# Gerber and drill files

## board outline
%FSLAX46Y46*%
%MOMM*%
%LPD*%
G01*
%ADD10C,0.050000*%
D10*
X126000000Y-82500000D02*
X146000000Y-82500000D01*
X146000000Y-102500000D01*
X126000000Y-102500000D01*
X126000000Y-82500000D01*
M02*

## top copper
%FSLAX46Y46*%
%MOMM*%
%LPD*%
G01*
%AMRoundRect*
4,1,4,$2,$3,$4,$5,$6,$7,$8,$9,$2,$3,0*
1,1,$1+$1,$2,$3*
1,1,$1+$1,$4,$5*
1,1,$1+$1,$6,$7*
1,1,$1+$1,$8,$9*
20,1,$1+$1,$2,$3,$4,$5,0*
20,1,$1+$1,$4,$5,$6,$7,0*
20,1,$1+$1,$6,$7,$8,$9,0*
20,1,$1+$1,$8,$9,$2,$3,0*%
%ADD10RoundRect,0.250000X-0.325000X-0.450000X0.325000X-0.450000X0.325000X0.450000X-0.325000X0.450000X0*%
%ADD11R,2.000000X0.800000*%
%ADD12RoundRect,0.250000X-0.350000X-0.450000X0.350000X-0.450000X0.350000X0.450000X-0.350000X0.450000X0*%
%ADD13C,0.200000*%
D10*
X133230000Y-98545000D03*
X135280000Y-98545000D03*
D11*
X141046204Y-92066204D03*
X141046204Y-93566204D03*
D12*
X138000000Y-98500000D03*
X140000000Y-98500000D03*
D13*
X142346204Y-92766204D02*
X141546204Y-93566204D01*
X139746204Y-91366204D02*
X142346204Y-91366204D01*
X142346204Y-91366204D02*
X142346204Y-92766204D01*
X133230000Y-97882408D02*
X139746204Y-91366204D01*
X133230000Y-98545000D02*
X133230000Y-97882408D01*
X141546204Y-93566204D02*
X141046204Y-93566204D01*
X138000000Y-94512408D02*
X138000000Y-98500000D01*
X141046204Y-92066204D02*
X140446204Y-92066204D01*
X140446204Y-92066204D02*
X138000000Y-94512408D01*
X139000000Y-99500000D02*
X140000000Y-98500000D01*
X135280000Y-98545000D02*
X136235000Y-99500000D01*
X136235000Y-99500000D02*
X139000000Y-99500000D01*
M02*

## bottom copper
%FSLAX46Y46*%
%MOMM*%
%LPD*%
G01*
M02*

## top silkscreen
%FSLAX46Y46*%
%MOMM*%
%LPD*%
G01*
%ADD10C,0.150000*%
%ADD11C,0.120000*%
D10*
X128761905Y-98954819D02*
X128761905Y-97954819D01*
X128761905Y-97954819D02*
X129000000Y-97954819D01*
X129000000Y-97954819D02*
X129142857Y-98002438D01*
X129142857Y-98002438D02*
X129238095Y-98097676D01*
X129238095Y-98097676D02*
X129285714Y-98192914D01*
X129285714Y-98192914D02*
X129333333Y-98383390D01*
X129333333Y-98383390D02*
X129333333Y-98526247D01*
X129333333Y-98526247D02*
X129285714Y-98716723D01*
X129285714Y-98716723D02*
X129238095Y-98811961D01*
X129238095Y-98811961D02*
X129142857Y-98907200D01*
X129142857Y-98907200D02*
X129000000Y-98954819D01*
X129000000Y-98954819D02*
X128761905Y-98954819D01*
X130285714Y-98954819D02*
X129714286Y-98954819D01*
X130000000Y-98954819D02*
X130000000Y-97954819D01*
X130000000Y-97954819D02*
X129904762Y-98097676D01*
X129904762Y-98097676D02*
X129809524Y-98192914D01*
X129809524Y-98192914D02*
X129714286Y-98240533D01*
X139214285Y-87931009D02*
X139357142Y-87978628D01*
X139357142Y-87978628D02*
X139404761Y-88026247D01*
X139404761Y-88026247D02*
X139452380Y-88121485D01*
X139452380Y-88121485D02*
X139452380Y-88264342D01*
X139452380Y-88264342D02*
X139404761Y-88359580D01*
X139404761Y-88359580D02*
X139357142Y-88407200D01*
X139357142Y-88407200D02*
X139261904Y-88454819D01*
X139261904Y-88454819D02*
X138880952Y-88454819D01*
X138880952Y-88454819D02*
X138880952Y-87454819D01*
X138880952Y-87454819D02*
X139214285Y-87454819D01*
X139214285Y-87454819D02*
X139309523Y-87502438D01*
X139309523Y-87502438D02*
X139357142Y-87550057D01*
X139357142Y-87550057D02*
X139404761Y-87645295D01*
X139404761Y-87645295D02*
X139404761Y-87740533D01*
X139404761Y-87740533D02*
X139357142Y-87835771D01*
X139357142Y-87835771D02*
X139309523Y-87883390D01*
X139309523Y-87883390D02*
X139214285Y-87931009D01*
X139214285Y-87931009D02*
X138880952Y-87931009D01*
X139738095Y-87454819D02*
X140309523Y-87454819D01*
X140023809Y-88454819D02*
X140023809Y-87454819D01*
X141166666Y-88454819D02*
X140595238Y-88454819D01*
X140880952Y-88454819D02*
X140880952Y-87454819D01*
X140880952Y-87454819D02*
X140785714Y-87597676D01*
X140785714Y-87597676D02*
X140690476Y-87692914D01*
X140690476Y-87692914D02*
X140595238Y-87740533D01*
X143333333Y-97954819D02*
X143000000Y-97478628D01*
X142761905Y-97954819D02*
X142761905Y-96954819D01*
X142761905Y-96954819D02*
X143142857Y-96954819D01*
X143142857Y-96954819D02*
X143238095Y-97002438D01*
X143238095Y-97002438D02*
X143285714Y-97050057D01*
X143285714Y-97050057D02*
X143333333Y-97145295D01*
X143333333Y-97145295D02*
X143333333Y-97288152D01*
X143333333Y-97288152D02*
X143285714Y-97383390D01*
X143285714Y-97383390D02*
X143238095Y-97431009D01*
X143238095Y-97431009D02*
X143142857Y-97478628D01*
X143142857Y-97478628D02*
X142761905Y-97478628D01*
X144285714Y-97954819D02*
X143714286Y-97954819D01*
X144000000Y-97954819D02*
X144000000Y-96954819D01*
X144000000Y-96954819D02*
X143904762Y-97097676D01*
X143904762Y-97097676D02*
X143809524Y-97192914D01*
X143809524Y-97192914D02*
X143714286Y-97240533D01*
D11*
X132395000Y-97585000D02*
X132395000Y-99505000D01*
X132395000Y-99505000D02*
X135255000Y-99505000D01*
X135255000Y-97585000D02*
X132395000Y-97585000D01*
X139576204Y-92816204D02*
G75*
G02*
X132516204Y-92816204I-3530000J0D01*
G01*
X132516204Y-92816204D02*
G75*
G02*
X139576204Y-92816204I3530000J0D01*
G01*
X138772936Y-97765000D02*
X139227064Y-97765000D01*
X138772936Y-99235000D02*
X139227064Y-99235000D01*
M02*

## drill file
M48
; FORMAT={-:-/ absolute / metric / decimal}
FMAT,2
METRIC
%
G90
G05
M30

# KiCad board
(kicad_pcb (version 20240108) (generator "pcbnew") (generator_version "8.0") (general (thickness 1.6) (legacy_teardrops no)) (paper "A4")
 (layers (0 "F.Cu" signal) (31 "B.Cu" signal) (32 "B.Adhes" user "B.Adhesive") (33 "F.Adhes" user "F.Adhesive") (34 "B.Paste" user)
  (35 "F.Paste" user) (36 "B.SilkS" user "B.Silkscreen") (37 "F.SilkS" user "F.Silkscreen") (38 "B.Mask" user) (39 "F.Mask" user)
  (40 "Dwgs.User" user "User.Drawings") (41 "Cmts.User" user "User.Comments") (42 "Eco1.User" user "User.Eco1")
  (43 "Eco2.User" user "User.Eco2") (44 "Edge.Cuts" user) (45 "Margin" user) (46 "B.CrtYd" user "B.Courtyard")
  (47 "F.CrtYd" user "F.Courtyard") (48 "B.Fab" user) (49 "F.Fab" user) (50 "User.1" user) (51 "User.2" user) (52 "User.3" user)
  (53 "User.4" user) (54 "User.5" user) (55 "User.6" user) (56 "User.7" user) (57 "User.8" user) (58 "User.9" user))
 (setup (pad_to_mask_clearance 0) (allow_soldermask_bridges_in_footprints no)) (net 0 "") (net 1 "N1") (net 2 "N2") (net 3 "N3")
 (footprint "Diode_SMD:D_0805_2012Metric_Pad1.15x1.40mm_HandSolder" (layer "F.Cu") (at 134.255 98.545)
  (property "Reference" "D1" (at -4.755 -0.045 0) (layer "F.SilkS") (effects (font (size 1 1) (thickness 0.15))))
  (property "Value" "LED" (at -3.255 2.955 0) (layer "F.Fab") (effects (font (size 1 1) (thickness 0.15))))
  (fp_line (start -1.86 -0.96) (end -1.86 0.96) (stroke (width 0.12) (type solid)) (layer "F.SilkS"))
  (fp_line (start -1.86 0.96) (end 1 0.96) (stroke (width 0.12) (type solid)) (layer "F.SilkS"))
  (fp_line (start 1 -0.96) (end -1.86 -0.96) (stroke (width 0.12) (type solid)) (layer "F.SilkS"))
  (pad "1" smd roundrect (at -1.025 0) (size 1.15 1.4) (layers "F.Cu" "F.Paste" "F.Mask") (roundrect_rratio 0.217391) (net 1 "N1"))
  (pad "2" smd roundrect (at 1.025 0) (size 1.15 1.4) (layers "F.Cu" "F.Paste" "F.Mask") (roundrect_rratio 0.217391) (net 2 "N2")))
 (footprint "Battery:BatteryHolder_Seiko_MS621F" (layer "F.Cu") (at 141.046204 92.816204)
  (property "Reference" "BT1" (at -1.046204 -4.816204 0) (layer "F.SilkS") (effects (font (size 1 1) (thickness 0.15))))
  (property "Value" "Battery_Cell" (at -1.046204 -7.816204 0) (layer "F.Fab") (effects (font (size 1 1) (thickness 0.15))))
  (fp_circle (center -5 0) (end -1.47 0) (stroke (width 0.12) (type solid)) (fill none) (layer "F.SilkS"))
  (pad "1" smd rect (at 0 -0.75) (size 2 0.8) (layers "F.Cu" "F.Paste" "F.Mask") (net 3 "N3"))
  (pad "2" smd rect (at 0 0.75) (size 2 0.8) (layers "F.Cu" "F.Paste" "F.Mask") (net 1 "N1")))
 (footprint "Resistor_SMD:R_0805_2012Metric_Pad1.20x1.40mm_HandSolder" (layer "F.Cu") (at 139 98.5)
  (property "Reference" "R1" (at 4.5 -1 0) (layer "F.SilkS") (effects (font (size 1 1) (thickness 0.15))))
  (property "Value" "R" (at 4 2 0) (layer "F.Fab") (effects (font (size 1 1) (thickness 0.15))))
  (fp_line (start -0.227064 -0.735) (end 0.227064 -0.735) (stroke (width 0.12) (type solid)) (layer "F.SilkS"))
  (fp_line (start -0.227064 0.735) (end 0.227064 0.735) (stroke (width 0.12) (type solid)) (layer "F.SilkS"))
  (pad "1" smd roundrect (at -1 0) (size 1.2 1.4) (layers "F.Cu" "F.Paste" "F.Mask") (roundrect_rratio 0.208333) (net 3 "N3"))
  (pad "2" smd roundrect (at 1 0) (size 1.2 1.4) (layers "F.Cu" "F.Paste" "F.Mask") (roundrect_rratio 0.208333) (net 2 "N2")))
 (gr_rect (start 126 82.5) (end 146 102.5) (stroke (width 0.05) (type default)) (fill none) (layer "Edge.Cuts"))
 (segment (start 142.346204 92.766204) (end 141.546204 93.566204) (width 0.2) (layer "F.Cu") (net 1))
 (segment (start 139.746204 91.366204) (end 142.346204 91.366204) (width 0.2) (layer "F.Cu") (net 1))
 (segment (start 142.346204 91.366204) (end 142.346204 92.766204) (width 0.2) (layer "F.Cu") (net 1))
 (segment (start 133.23 97.882408) (end 139.746204 91.366204) (width 0.2) (layer "F.Cu") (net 1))
 (segment (start 133.23 98.545) (end 133.23 97.882408) (width 0.2) (layer "F.Cu") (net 1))
 (segment (start 141.546204 93.566204) (end 141.046204 93.566204) (width 0.2) (layer "F.Cu") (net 1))
 (segment (start 138 94.512408) (end 138 98.5) (width 0.2) (layer "F.Cu") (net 3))
 (segment (start 141.046204 92.066204) (end 140.446204 92.066204) (width 0.2) (layer "F.Cu") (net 3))
 (segment (start 140.446204 92.066204) (end 138 94.512408) (width 0.2) (layer "F.Cu") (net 3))
 (segment (start 139 99.5) (end 140 98.5) (width 0.2) (layer "F.Cu") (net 2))
 (segment (start 135.28 98.545) (end 136.235 99.5) (width 0.2) (layer "F.Cu") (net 2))
 (segment (start 136.235 99.5) (end 139 99.5) (width 0.2) (layer "F.Cu") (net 2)))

